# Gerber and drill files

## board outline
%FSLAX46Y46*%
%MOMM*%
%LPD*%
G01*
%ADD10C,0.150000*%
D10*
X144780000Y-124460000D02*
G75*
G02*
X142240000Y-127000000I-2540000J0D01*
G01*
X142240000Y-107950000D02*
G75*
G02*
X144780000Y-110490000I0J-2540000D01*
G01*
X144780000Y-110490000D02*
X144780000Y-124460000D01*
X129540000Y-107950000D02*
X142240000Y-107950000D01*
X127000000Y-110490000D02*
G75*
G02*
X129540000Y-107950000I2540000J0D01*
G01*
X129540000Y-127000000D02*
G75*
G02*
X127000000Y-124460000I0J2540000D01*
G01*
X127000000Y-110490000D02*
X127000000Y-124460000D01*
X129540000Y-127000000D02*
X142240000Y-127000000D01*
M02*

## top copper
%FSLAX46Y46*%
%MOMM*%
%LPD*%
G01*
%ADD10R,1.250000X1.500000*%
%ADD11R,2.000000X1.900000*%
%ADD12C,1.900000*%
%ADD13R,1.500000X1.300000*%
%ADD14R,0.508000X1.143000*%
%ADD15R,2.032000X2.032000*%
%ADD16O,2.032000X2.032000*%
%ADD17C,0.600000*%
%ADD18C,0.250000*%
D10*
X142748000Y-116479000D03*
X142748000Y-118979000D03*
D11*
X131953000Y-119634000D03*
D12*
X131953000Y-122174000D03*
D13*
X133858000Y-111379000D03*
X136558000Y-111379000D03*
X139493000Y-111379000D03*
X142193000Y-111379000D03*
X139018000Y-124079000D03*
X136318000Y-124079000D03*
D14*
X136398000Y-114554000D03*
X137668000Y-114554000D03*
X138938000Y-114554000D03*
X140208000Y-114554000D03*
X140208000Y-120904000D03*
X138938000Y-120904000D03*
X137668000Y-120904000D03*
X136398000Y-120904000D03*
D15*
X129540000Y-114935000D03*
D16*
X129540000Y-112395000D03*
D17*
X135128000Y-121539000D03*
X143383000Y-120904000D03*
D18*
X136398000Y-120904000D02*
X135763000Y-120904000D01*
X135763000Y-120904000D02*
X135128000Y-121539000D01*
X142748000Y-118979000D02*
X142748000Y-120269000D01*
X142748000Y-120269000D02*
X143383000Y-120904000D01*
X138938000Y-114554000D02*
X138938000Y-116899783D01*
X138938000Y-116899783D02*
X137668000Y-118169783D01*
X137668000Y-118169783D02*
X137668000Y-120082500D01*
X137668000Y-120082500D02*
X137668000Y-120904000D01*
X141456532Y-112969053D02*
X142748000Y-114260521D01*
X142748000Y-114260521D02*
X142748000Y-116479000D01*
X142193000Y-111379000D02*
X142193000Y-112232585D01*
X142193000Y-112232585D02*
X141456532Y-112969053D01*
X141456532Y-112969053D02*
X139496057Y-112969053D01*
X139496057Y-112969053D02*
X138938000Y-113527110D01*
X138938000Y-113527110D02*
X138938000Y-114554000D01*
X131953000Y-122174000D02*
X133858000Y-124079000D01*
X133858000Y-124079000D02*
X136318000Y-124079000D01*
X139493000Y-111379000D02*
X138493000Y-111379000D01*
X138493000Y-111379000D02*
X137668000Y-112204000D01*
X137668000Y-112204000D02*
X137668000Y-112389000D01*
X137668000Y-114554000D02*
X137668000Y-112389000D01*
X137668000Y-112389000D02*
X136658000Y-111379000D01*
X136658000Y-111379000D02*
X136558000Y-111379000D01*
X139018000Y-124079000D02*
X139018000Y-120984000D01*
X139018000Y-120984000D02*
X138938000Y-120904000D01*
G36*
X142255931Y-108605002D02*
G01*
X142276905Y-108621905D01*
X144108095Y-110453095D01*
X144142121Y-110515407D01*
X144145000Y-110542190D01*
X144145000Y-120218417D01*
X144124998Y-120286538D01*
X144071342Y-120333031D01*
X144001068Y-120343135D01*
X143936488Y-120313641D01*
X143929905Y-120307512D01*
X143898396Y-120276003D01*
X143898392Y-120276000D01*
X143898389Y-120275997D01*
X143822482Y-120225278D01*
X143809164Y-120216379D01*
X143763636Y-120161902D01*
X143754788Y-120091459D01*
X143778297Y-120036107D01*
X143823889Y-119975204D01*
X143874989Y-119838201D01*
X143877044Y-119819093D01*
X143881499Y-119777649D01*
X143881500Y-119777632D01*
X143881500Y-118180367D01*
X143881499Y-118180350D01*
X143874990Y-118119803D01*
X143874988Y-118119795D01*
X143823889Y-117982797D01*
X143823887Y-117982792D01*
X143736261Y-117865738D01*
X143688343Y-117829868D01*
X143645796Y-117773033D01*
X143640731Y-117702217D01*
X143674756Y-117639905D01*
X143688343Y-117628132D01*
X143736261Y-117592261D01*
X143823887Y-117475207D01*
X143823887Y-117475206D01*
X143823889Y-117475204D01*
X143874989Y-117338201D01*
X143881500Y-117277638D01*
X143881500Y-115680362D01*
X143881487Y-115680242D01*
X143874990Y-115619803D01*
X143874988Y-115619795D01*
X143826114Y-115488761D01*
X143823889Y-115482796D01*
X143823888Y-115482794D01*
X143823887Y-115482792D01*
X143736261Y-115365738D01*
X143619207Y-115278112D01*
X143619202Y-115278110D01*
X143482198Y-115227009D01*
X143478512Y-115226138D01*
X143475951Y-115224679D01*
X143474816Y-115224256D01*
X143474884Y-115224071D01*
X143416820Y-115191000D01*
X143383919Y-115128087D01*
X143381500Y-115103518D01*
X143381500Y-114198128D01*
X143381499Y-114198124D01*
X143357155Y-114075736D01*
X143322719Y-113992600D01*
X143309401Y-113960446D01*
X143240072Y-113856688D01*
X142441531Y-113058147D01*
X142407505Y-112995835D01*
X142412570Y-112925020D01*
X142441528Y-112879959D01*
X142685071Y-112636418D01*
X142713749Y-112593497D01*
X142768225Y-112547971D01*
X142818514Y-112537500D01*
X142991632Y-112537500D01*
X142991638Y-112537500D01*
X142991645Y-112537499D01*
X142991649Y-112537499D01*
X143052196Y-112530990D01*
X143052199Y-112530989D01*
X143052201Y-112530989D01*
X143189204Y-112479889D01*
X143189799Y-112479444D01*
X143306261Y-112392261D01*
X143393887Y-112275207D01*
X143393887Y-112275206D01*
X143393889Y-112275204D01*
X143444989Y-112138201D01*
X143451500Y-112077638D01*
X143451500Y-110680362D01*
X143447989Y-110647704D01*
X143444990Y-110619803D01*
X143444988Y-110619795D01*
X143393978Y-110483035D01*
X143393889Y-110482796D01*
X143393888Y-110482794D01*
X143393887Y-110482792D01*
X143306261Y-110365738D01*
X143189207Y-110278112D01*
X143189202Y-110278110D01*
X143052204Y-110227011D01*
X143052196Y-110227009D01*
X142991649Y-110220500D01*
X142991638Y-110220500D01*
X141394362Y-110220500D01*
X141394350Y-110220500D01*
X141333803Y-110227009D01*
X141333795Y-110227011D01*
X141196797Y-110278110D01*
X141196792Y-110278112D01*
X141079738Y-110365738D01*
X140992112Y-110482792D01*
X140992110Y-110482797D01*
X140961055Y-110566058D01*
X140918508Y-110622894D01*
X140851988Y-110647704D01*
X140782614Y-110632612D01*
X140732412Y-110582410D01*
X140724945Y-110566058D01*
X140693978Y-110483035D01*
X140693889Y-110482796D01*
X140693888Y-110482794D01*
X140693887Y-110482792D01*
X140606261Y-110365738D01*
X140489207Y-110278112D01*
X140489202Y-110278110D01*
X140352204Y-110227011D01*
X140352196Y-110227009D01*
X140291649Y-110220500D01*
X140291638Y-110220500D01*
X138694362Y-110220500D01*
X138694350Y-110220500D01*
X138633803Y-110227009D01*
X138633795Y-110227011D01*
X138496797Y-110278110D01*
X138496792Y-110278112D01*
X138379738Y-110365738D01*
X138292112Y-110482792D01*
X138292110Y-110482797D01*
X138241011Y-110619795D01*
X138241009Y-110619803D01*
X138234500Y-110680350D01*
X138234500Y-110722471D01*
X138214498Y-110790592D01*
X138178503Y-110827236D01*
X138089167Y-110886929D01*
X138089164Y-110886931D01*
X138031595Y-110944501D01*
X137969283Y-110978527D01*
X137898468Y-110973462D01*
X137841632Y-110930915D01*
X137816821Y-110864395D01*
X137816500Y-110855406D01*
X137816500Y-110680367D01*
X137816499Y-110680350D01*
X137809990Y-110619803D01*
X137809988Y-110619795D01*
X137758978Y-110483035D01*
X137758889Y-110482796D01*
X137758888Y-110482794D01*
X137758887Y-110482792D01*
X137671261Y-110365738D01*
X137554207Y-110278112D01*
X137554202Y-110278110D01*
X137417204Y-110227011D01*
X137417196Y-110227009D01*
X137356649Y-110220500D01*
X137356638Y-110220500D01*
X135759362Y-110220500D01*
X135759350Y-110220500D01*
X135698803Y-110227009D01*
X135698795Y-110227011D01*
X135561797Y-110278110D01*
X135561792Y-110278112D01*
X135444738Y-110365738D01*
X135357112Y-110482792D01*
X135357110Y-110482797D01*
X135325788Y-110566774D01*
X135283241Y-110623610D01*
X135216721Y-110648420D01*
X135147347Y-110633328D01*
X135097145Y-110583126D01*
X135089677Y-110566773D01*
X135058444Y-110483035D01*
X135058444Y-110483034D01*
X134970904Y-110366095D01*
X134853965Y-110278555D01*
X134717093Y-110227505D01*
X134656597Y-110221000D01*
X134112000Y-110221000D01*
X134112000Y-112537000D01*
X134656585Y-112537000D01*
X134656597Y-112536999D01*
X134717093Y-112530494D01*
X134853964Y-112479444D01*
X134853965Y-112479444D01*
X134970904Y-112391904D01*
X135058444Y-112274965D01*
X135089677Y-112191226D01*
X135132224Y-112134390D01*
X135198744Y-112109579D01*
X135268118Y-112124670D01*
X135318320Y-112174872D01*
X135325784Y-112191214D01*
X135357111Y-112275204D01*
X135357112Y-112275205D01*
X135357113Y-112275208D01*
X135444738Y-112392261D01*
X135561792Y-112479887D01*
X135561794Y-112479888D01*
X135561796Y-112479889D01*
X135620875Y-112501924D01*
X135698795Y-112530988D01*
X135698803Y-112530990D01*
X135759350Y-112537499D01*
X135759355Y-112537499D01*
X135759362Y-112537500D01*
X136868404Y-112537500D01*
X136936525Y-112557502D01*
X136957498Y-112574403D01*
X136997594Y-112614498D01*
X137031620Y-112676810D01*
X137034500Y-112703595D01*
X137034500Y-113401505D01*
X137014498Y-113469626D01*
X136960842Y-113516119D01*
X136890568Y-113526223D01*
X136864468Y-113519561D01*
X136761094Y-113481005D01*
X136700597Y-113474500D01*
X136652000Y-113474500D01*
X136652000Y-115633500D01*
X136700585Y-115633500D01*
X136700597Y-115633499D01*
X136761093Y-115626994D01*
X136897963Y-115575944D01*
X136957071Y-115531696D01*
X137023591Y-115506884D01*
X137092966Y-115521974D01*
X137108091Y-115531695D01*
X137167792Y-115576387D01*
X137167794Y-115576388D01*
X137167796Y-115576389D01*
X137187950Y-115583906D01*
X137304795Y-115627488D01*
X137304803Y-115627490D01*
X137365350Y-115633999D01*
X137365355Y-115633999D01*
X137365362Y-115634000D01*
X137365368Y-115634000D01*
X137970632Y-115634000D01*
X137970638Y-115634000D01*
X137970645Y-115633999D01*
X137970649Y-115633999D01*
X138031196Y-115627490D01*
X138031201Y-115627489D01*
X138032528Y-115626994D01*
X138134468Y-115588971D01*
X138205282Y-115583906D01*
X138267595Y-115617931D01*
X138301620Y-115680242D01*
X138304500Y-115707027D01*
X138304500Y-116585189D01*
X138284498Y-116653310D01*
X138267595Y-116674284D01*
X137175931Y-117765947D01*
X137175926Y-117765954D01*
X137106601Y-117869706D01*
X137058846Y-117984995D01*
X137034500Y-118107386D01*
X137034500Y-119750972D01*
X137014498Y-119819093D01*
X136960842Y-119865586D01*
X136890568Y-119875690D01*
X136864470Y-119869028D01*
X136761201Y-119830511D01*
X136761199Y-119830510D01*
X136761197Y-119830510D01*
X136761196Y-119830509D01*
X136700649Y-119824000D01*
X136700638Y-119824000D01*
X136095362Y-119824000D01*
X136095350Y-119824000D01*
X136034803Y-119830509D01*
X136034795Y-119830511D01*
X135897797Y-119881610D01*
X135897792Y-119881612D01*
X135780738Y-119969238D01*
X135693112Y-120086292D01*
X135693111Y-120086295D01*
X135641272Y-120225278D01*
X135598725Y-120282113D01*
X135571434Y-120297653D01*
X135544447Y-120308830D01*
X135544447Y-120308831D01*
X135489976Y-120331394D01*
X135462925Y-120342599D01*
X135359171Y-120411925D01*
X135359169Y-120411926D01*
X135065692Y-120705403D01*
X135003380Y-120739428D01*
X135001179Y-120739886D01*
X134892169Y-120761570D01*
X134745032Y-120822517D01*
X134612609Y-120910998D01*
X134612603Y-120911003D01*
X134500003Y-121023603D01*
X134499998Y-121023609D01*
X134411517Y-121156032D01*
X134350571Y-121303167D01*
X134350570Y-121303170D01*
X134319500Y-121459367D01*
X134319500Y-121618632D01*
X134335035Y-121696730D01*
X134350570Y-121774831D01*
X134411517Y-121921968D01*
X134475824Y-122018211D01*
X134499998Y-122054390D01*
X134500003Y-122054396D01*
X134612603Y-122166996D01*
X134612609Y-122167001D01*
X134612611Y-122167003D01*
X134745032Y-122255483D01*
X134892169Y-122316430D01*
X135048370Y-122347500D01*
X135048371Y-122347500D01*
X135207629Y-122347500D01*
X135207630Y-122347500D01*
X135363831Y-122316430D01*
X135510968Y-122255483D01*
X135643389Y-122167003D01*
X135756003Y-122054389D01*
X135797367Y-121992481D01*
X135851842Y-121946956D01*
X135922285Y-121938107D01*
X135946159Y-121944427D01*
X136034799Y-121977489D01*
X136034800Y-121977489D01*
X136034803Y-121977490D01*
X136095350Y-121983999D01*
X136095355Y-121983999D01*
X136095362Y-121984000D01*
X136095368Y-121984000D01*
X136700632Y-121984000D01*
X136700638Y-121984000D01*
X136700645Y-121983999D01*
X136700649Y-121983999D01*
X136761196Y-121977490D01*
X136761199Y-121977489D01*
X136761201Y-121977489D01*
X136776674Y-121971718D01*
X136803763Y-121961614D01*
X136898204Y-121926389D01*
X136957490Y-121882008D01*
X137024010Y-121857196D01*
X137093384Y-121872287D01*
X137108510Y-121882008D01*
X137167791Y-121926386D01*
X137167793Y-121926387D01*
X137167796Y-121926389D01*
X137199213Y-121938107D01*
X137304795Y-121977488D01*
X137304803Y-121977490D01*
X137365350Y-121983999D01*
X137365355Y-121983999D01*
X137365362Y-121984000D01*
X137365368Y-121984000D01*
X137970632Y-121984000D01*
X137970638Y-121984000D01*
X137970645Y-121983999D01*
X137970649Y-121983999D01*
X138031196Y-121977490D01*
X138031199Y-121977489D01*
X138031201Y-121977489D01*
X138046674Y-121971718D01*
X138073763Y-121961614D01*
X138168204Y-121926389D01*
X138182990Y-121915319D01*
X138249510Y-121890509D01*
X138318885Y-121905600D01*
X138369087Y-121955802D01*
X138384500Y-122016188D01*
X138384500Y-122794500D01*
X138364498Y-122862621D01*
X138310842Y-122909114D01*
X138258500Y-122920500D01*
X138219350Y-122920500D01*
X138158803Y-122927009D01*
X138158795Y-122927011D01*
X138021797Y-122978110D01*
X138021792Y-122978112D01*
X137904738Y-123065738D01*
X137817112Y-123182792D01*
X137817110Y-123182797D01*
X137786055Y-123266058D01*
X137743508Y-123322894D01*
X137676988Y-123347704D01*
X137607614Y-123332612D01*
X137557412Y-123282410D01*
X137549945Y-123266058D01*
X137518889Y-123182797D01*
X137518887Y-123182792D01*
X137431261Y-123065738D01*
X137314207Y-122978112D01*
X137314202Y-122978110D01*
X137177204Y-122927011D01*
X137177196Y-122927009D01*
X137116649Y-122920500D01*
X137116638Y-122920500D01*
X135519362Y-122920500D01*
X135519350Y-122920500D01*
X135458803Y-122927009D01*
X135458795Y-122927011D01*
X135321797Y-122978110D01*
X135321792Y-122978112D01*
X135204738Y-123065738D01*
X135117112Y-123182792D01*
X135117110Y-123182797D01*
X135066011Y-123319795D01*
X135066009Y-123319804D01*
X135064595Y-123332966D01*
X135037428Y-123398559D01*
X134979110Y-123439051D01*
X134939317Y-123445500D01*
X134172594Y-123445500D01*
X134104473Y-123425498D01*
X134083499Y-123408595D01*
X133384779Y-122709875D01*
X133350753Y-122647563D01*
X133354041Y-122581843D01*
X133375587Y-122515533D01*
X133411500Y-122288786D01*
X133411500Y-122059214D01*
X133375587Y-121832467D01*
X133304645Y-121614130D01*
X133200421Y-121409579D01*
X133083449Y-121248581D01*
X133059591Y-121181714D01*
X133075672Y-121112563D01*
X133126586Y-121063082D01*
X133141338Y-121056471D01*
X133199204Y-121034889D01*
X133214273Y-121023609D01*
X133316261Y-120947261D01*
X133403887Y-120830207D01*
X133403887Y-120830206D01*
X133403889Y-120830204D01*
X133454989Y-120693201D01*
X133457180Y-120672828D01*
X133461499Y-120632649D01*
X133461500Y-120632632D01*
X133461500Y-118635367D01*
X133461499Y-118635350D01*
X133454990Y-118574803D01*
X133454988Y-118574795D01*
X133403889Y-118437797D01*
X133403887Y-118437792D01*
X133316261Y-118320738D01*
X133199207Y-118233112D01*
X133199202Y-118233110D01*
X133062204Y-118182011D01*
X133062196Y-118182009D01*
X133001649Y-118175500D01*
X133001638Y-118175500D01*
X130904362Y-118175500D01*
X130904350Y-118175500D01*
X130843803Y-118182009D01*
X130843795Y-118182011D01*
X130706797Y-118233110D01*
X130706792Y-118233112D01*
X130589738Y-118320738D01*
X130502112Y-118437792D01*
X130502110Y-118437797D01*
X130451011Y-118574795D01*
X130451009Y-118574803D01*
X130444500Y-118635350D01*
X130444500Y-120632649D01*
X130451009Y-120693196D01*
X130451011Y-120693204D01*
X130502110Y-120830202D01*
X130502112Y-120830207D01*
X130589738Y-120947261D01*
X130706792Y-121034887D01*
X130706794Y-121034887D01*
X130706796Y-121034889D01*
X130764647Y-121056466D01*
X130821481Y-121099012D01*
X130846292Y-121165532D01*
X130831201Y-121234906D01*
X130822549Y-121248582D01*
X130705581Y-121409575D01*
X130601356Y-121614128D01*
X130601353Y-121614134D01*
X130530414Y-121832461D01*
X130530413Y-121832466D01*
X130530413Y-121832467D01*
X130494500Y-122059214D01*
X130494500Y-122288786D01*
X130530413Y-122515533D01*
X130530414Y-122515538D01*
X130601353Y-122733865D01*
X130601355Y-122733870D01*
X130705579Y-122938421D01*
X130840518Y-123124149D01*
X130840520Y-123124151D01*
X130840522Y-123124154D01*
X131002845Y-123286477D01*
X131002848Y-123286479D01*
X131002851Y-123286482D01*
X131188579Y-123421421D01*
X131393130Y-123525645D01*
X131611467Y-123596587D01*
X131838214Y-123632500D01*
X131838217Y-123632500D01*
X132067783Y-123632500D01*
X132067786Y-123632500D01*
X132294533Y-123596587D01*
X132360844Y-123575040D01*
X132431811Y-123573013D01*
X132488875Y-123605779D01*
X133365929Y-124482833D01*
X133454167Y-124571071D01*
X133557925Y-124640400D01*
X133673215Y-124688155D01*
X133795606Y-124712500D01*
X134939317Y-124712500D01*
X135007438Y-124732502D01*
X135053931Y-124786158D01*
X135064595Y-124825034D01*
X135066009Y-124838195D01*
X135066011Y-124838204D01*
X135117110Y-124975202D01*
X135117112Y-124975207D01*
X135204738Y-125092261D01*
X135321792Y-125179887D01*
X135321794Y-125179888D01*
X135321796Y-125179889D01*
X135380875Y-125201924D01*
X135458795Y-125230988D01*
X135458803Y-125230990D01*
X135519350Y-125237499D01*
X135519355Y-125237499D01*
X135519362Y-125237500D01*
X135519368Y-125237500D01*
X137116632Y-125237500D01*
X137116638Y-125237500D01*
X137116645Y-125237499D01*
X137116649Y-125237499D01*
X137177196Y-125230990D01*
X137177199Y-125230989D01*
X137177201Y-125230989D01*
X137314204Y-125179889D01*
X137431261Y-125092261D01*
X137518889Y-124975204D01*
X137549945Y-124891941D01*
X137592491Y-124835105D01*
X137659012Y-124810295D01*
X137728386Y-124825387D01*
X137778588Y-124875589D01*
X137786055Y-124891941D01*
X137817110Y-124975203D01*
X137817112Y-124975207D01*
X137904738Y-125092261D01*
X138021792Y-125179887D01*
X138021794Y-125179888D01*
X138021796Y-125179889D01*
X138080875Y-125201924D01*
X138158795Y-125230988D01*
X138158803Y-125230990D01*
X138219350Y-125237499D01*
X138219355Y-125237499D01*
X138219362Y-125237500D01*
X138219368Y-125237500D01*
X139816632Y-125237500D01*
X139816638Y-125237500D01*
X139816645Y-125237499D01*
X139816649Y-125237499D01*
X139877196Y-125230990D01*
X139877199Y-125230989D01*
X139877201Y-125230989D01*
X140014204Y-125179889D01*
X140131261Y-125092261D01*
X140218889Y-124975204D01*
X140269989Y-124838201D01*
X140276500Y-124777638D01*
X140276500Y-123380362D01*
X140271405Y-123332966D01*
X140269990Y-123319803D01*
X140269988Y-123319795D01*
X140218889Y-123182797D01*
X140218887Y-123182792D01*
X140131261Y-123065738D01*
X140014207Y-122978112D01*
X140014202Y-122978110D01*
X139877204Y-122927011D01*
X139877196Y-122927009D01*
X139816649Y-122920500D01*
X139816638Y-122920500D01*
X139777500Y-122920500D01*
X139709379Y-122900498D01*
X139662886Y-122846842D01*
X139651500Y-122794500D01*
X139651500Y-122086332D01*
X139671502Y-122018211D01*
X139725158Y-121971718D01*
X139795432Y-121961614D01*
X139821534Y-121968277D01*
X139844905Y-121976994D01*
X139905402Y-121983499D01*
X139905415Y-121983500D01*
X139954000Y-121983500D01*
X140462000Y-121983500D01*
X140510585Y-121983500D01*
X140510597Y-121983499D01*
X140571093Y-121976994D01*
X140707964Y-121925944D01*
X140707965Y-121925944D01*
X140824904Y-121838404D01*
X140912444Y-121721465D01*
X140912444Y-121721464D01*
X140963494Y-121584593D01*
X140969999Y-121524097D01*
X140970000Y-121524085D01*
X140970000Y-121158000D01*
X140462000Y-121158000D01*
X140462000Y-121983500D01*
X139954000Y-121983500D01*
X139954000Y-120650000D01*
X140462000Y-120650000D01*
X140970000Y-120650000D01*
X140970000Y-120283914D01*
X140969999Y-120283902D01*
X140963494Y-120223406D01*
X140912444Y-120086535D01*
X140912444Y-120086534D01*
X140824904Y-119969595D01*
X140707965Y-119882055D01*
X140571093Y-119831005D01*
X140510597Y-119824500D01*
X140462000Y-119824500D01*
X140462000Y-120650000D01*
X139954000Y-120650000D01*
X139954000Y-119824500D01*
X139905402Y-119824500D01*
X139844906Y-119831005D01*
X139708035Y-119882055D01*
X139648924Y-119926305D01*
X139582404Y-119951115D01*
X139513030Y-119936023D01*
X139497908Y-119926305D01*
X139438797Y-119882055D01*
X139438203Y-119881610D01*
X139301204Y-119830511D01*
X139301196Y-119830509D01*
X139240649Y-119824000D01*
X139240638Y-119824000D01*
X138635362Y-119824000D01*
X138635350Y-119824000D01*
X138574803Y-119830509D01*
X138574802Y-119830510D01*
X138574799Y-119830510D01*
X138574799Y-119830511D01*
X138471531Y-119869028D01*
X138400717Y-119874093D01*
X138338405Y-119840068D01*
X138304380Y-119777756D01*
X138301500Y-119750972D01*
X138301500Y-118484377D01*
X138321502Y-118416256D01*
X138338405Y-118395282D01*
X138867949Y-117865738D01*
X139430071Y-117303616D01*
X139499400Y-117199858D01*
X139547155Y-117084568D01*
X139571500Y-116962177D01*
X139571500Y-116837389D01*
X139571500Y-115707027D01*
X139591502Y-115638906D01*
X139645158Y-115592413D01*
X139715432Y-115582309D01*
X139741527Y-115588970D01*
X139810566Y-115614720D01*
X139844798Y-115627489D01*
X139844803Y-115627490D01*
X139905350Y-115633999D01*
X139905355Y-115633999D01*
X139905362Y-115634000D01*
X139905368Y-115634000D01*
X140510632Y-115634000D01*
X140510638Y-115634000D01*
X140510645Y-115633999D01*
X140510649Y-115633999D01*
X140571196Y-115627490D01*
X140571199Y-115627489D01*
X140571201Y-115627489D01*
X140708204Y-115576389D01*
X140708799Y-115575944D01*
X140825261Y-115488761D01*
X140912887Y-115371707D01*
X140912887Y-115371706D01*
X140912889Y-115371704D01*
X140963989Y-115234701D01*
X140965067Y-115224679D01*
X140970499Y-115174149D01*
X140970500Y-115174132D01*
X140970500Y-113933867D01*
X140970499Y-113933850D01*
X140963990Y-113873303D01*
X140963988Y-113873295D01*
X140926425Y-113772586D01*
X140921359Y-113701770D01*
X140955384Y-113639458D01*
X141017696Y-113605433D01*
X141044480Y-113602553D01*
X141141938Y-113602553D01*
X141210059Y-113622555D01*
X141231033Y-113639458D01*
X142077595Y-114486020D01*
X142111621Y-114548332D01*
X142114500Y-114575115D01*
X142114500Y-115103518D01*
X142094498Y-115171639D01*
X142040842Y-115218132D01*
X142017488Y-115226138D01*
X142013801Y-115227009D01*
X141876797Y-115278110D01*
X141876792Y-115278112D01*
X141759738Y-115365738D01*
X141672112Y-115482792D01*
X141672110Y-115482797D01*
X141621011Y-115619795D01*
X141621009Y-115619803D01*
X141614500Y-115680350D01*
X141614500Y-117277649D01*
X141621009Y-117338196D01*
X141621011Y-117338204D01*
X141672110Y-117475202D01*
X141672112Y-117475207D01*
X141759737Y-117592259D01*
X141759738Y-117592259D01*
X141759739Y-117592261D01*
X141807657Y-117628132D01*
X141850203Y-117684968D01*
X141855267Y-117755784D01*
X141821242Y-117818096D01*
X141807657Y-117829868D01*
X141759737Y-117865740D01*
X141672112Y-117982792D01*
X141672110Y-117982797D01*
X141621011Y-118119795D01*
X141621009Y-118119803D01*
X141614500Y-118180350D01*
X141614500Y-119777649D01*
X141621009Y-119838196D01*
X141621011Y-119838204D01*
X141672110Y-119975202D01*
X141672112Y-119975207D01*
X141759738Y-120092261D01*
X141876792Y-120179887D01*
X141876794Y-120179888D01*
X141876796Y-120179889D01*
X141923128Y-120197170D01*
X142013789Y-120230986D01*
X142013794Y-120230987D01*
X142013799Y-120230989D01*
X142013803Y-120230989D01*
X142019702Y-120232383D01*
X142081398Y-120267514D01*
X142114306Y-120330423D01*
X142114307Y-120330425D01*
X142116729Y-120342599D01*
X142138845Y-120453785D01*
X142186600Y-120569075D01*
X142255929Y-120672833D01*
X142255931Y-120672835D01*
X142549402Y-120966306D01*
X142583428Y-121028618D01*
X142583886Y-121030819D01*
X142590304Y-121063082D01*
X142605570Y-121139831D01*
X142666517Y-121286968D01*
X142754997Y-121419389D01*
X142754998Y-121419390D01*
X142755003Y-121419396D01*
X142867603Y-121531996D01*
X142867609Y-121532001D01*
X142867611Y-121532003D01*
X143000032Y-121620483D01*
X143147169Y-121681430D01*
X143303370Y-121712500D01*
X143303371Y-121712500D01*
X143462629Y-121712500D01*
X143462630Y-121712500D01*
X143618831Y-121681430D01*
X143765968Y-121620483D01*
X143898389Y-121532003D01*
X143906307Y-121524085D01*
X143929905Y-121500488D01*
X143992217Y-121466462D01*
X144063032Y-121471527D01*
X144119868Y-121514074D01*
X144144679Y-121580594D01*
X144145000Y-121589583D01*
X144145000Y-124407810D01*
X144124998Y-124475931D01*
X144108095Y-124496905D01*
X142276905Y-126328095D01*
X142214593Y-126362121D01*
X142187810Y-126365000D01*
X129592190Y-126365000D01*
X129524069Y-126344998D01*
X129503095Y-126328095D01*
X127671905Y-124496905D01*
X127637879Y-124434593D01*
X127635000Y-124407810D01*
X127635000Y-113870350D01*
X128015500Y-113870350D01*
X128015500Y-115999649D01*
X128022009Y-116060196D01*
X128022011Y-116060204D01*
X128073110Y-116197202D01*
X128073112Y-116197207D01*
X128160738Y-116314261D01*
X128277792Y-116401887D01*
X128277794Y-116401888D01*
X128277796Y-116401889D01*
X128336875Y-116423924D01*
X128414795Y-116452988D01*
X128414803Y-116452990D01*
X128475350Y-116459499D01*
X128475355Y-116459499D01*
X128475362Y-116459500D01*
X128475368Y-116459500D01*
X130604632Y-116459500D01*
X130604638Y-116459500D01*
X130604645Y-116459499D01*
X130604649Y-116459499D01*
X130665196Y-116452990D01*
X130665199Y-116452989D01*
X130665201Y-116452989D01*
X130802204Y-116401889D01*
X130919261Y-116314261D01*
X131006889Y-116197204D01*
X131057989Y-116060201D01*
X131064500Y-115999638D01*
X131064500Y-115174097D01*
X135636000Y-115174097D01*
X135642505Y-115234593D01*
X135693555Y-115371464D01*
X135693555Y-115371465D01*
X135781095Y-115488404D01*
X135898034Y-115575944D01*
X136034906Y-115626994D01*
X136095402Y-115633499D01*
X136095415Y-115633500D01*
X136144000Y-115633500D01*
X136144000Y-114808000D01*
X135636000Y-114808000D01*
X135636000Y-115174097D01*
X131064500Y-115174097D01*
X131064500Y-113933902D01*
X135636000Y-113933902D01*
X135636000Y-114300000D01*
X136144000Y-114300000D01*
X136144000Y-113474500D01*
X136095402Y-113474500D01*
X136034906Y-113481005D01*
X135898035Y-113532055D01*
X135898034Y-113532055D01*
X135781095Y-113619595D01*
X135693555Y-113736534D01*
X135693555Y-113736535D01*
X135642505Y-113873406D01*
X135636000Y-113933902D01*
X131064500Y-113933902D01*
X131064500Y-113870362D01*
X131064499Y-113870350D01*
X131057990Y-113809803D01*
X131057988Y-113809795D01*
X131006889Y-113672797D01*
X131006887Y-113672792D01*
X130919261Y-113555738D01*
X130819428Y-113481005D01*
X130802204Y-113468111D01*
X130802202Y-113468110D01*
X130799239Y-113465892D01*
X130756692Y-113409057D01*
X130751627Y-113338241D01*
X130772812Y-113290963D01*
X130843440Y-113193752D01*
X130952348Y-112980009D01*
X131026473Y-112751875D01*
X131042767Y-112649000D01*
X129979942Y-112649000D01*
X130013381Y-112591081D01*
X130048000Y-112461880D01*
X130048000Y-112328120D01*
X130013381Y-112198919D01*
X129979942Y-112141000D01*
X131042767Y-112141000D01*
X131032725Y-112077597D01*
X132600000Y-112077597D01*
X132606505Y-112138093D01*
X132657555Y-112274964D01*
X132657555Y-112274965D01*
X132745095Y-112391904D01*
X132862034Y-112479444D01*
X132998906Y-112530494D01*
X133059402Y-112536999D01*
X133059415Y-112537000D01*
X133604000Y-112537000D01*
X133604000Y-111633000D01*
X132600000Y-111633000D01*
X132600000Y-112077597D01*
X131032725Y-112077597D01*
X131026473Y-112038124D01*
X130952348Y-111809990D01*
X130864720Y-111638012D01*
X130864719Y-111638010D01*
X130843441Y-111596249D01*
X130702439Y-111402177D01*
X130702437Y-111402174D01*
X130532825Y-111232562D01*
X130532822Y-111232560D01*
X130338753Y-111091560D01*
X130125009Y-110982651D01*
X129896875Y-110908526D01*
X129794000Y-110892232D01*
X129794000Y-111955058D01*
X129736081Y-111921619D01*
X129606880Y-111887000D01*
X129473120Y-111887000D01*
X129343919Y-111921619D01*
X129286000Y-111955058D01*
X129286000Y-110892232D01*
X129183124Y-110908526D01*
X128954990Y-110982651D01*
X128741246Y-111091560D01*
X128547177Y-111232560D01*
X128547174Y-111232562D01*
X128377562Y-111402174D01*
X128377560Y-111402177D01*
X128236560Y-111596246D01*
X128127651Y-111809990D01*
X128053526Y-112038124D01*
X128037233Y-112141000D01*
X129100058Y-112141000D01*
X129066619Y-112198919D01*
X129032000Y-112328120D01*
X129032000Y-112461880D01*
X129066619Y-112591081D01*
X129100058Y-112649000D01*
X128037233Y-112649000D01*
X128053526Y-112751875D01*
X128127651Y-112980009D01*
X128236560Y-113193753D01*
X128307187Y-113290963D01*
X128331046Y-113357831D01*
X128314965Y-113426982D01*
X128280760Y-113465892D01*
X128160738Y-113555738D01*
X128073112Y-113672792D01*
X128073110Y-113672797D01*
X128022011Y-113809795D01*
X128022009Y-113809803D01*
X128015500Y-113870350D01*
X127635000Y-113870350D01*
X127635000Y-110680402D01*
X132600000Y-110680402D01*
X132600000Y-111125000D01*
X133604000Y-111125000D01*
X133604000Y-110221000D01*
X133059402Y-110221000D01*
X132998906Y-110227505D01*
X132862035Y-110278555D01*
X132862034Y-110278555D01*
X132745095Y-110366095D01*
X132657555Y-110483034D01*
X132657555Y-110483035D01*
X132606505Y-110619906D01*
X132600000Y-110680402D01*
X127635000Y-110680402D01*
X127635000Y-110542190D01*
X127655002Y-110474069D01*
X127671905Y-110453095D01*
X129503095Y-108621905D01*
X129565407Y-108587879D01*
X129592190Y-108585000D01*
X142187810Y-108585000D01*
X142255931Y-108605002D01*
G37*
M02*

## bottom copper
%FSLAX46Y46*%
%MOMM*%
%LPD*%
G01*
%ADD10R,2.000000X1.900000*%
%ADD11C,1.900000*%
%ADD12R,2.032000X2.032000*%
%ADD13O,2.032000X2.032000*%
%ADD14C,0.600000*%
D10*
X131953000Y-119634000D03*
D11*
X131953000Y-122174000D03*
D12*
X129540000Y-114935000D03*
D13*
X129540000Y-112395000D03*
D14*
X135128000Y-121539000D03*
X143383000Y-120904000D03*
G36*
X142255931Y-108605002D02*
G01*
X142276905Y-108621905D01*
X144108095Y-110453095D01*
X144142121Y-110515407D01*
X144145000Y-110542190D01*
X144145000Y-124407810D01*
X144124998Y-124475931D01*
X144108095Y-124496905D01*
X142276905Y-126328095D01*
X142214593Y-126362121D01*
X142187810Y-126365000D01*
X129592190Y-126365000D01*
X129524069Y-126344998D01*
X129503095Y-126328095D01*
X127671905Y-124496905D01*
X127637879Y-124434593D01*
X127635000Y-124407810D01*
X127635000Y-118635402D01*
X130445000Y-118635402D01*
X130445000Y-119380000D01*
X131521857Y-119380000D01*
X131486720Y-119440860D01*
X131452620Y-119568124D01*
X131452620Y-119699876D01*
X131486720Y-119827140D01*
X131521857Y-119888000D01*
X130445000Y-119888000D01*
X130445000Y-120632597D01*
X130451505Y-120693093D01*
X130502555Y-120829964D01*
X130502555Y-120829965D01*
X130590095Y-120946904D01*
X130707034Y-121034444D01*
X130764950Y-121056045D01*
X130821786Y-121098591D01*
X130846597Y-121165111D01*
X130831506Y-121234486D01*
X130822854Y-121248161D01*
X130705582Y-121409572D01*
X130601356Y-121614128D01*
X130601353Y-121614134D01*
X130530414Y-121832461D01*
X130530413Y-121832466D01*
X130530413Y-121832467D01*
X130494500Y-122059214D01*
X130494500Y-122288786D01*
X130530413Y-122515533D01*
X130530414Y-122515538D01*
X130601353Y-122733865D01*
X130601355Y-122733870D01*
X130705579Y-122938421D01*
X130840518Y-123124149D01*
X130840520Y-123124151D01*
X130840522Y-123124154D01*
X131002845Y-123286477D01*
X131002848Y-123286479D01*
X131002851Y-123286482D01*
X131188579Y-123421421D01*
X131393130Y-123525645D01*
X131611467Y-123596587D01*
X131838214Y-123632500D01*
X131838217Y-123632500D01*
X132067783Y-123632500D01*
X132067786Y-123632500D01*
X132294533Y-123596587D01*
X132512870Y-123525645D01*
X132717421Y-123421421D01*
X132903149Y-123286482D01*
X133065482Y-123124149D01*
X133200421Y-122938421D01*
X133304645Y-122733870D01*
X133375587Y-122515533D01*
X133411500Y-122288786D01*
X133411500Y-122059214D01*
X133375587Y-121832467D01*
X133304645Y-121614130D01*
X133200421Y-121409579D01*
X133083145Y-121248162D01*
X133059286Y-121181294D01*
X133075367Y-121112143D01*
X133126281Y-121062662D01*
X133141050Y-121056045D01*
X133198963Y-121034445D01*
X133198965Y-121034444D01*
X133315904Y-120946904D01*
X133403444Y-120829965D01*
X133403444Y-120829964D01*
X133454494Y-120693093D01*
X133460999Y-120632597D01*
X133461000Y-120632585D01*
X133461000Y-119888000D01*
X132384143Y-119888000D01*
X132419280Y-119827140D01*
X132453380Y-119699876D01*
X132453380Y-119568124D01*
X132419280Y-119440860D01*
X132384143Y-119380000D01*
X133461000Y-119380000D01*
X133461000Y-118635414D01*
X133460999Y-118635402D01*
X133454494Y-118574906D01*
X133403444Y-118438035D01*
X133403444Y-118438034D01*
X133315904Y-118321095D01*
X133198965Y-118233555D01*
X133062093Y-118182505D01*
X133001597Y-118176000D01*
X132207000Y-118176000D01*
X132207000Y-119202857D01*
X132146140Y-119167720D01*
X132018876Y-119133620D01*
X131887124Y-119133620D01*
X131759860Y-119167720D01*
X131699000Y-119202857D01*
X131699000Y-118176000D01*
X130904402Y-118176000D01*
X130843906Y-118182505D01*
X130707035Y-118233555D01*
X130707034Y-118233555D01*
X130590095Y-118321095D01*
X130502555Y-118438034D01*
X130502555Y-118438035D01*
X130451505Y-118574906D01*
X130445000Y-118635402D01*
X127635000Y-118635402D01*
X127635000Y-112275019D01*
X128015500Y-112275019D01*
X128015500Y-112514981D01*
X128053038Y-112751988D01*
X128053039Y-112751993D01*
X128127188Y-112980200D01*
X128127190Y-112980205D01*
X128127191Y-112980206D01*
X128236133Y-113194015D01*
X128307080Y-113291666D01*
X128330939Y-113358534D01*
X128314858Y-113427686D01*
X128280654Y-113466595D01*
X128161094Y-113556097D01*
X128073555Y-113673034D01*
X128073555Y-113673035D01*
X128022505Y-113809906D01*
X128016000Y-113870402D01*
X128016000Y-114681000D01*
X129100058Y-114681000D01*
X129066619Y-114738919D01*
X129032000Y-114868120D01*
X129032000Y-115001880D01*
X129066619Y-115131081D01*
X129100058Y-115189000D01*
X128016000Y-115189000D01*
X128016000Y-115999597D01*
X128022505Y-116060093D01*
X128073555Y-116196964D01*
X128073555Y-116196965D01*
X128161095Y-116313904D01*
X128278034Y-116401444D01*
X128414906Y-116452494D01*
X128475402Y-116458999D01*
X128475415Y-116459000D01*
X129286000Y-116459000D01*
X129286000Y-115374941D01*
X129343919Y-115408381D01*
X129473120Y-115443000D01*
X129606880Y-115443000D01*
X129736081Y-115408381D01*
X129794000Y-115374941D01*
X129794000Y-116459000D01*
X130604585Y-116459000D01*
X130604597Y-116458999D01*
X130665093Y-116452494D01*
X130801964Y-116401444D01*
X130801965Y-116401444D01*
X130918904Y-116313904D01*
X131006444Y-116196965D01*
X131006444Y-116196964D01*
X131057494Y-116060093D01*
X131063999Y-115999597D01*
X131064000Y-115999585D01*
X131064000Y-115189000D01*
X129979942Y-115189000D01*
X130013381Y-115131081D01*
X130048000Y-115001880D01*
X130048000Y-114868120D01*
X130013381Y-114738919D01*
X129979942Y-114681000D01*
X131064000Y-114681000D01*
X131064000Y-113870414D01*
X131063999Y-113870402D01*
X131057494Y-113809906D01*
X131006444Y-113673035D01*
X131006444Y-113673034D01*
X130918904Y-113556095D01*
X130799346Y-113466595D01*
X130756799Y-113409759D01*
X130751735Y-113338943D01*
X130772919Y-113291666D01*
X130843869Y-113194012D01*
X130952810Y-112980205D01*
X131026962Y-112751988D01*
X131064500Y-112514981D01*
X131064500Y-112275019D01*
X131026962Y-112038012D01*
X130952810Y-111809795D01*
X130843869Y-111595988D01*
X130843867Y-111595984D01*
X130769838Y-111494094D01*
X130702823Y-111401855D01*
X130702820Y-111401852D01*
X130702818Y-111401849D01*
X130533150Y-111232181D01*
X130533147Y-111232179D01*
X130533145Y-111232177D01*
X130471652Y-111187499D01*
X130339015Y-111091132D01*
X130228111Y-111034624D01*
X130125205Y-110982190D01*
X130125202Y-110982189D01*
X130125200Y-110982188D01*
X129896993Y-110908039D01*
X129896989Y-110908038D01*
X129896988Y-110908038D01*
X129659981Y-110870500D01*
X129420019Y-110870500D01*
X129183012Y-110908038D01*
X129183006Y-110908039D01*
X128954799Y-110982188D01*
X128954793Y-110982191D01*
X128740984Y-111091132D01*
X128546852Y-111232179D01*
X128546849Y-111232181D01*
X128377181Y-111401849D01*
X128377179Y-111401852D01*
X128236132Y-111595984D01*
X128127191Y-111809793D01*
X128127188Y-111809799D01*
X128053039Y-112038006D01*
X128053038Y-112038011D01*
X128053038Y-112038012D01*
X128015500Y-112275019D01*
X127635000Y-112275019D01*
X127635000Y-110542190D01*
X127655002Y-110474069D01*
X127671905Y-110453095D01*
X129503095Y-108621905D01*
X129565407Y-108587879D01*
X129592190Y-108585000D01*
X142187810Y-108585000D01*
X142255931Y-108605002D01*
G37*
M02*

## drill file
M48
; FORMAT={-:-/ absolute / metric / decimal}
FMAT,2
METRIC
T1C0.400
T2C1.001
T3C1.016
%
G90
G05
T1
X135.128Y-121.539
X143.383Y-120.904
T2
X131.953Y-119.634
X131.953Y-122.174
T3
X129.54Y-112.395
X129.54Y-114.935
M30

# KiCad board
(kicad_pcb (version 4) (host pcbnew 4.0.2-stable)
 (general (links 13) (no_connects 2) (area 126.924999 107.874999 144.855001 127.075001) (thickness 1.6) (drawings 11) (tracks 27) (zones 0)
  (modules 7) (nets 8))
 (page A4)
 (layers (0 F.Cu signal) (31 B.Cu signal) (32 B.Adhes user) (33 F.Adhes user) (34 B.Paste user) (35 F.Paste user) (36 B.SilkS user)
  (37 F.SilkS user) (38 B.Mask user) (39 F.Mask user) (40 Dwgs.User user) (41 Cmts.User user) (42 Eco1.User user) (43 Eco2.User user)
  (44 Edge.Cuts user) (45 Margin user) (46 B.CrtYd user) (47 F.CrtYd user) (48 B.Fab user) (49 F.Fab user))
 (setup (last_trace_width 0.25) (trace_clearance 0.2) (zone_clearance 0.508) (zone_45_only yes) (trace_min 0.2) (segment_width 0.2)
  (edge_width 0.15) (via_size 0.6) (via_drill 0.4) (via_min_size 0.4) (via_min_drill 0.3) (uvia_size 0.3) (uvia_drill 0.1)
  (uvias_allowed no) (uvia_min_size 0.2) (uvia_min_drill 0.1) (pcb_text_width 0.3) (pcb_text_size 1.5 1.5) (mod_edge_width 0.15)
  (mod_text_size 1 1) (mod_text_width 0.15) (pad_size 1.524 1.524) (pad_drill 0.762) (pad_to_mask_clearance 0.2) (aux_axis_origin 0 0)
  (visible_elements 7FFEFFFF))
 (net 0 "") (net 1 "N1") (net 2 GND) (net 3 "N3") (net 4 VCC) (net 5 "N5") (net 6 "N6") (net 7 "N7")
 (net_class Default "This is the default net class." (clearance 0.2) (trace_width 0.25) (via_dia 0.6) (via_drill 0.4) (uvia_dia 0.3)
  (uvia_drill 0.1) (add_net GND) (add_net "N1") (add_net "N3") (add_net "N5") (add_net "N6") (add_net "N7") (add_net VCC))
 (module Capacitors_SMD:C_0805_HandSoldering (layer F.Cu) (at 142.748 117.729 270)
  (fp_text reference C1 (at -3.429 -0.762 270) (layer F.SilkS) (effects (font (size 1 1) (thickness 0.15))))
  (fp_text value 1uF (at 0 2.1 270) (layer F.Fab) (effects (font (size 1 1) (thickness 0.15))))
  (pad 1 smd rect (at -1.25 0 270) (size 1.5 1.25) (layers F.Cu F.Paste F.Mask) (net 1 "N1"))
  (pad 2 smd rect (at 1.25 0 270) (size 1.5 1.25) (layers F.Cu F.Paste F.Mask) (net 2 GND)))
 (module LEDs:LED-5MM (layer F.Cu) (at 131.953 119.634 270)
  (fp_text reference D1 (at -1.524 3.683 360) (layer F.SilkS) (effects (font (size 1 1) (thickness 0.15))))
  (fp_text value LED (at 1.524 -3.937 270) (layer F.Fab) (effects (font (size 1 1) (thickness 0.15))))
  (pad 1 thru_hole rect (at 0 0) (size 2 1.9) (drill 1.00076) (layers *.Cu *.Mask F.SilkS) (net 2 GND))
  (pad 2 thru_hole circle (at 2.54 0 270) (size 1.9 1.9) (drill 1.00076) (layers *.Cu *.Mask F.SilkS) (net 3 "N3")))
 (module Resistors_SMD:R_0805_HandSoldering (layer F.Cu) (at 135.208 111.379)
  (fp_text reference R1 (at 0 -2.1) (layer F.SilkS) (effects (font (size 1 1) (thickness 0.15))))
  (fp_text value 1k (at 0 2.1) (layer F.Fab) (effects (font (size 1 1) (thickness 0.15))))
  (pad 1 smd rect (at -1.35 0) (size 1.5 1.3) (layers F.Cu F.Paste F.Mask) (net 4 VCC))
  (pad 2 smd rect (at 1.35 0) (size 1.5 1.3) (layers F.Cu F.Paste F.Mask) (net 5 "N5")))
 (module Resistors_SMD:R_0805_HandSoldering (layer F.Cu) (at 140.843 111.379)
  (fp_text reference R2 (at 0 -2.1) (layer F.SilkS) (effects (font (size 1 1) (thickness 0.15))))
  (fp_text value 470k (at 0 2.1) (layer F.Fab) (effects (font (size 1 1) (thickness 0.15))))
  (pad 1 smd rect (at -1.35 0) (size 1.5 1.3) (layers F.Cu F.Paste F.Mask) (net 5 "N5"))
  (pad 2 smd rect (at 1.35 0) (size 1.5 1.3) (layers F.Cu F.Paste F.Mask) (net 1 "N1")))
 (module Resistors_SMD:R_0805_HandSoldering (layer F.Cu) (at 137.668 124.079 180)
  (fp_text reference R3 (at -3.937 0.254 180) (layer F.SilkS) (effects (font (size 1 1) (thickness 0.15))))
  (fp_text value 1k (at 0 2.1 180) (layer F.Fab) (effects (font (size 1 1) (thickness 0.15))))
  (pad 1 smd rect (at -1.35 0 180) (size 1.5 1.3) (layers F.Cu F.Paste F.Mask) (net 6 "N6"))
  (pad 2 smd rect (at 1.35 0 180) (size 1.5 1.3) (layers F.Cu F.Paste F.Mask) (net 3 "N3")))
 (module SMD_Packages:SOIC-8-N (layer F.Cu) (at 138.303 117.729)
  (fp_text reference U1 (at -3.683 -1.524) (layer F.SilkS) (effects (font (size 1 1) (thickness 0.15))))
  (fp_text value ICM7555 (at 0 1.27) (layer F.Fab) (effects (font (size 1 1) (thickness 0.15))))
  (pad 8 smd rect (at -1.905 -3.175) (size 0.508 1.143) (layers F.Cu F.Paste F.Mask) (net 4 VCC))
  (pad 7 smd rect (at -0.635 -3.175) (size 0.508 1.143) (layers F.Cu F.Paste F.Mask) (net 5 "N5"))
  (pad 6 smd rect (at 0.635 -3.175) (size 0.508 1.143) (layers F.Cu F.Paste F.Mask) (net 1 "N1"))
  (pad 5 smd rect (at 1.905 -3.175) (size 0.508 1.143) (layers F.Cu F.Paste F.Mask) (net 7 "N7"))
  (pad 4 smd rect (at 1.905 3.175) (size 0.508 1.143) (layers F.Cu F.Paste F.Mask) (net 4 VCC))
  (pad 3 smd rect (at 0.635 3.175) (size 0.508 1.143) (layers F.Cu F.Paste F.Mask) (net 6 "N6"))
  (pad 2 smd rect (at -0.635 3.175) (size 0.508 1.143) (layers F.Cu F.Paste F.Mask) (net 1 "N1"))
  (pad 1 smd rect (at -1.905 3.175) (size 0.508 1.143) (layers F.Cu F.Paste F.Mask) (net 2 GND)))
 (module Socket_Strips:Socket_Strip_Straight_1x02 (layer F.Cu) (at 129.54 114.935 90)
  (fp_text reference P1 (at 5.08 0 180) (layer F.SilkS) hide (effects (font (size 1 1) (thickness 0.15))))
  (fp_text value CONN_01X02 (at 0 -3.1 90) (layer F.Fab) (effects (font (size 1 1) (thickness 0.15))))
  (pad 1 thru_hole rect (at 0 0 90) (size 2.032 2.032) (drill 1.016) (layers *.Cu *.Mask F.SilkS) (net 2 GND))
  (pad 2 thru_hole oval (at 2.54 0 90) (size 2.032 2.032) (drill 1.016) (layers *.Cu *.Mask F.SilkS) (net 4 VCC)))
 (gr_arc (start 142.24 124.46) (end 144.78 124.46) (angle 90) (layer Edge.Cuts) (width 0.15))
 (gr_arc (start 142.24 110.49) (end 142.24 107.95) (angle 90) (layer Edge.Cuts) (width 0.15))
 (gr_line (start 144.78 110.49) (end 144.78 124.46) (layer Edge.Cuts) (width 0.15))
 (gr_line (start 129.54 107.95) (end 142.24 107.95) (layer Edge.Cuts) (width 0.15))
 (gr_arc (start 129.54 110.49) (end 127 110.49) (angle 90) (layer Edge.Cuts) (width 0.15))
 (gr_arc (start 129.54 124.46) (end 129.54 127) (angle 90) (layer Edge.Cuts) (width 0.15))
 (gr_line (start 127 110.49) (end 127 124.46) (layer Edge.Cuts) (width 0.15))
 (gr_line (start 129.54 127) (end 142.24 127) (layer Edge.Cuts) (width 0.15))
 (segment (start 136.398 120.904) (end 135.763 120.904) (width 0.25) (layer F.Cu) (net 2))
 (segment (start 135.763 120.904) (end 135.128 121.539) (width 0.25) (layer F.Cu) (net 2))
 (via (at 135.128 121.539) (size 0.6) (drill 0.4) (layers F.Cu B.Cu) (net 2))
 (segment (start 142.748 118.979) (end 142.748 120.269) (width 0.25) (layer F.Cu) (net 2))
 (via (at 143.383 120.904) (size 0.6) (drill 0.4) (layers F.Cu B.Cu) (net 2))
 (segment (start 142.748 120.269) (end 143.383 120.904) (width 0.25) (layer F.Cu) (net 2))
 (segment (start 138.938 114.554) (end 138.938 116.899783) (width 0.25) (layer F.Cu) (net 1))
 (segment (start 138.938 116.899783) (end 137.668 118.169783) (width 0.25) (layer F.Cu) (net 1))
 (segment (start 137.668 118.169783) (end 137.668 120.0825) (width 0.25) (layer F.Cu) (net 1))
 (segment (start 137.668 120.0825) (end 137.668 120.904) (width 0.25) (layer F.Cu) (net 1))
 (segment (start 141.456532 112.969053) (end 142.748 114.260521) (width 0.25) (layer F.Cu) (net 1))
 (segment (start 142.748 114.260521) (end 142.748 116.479) (width 0.25) (layer F.Cu) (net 1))
 (segment (start 142.193 111.379) (end 142.193 112.232585) (width 0.25) (layer F.Cu) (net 1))
 (segment (start 142.193 112.232585) (end 141.456532 112.969053) (width 0.25) (layer F.Cu) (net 1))
 (segment (start 141.456532 112.969053) (end 139.496057 112.969053) (width 0.25) (layer F.Cu) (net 1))
 (segment (start 139.496057 112.969053) (end 138.938 113.52711) (width 0.25) (layer F.Cu) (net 1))
 (segment (start 138.938 113.52711) (end 138.938 114.554) (width 0.25) (layer F.Cu) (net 1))
 (segment (start 131.953 122.174) (end 133.858 124.079) (width 0.25) (layer F.Cu) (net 3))
 (segment (start 133.858 124.079) (end 136.318 124.079) (width 0.25) (layer F.Cu) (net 3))
 (segment (start 139.493 111.379) (end 138.493 111.379) (width 0.25) (layer F.Cu) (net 5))
 (segment (start 138.493 111.379) (end 137.668 112.204) (width 0.25) (layer F.Cu) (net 5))
 (segment (start 137.668 112.204) (end 137.668 112.389) (width 0.25) (layer F.Cu) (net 5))
 (segment (start 137.668 114.554) (end 137.668 112.389) (width 0.25) (layer F.Cu) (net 5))
 (segment (start 137.668 112.389) (end 136.658 111.379) (width 0.25) (layer F.Cu) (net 5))
 (segment (start 136.658 111.379) (end 136.558 111.379) (width 0.25) (layer F.Cu) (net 5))
 (segment (start 139.018 124.079) (end 139.018 120.984) (width 0.25) (layer F.Cu) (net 6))
 (segment (start 139.018 120.984) (end 138.938 120.904) (width 0.25) (layer F.Cu) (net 6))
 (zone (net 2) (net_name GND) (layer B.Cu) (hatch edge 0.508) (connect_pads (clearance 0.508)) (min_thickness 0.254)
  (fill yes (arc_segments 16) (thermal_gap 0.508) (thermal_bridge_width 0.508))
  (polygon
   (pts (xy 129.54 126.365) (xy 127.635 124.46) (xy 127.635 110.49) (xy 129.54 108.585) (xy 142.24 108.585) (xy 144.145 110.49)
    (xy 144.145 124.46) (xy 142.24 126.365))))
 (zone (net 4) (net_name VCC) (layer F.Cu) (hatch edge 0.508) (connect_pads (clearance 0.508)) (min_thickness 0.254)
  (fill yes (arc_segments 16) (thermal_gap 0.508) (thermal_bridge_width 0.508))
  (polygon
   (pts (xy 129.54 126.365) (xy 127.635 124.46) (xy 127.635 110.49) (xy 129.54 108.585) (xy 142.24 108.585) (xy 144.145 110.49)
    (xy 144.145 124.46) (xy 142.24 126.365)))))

